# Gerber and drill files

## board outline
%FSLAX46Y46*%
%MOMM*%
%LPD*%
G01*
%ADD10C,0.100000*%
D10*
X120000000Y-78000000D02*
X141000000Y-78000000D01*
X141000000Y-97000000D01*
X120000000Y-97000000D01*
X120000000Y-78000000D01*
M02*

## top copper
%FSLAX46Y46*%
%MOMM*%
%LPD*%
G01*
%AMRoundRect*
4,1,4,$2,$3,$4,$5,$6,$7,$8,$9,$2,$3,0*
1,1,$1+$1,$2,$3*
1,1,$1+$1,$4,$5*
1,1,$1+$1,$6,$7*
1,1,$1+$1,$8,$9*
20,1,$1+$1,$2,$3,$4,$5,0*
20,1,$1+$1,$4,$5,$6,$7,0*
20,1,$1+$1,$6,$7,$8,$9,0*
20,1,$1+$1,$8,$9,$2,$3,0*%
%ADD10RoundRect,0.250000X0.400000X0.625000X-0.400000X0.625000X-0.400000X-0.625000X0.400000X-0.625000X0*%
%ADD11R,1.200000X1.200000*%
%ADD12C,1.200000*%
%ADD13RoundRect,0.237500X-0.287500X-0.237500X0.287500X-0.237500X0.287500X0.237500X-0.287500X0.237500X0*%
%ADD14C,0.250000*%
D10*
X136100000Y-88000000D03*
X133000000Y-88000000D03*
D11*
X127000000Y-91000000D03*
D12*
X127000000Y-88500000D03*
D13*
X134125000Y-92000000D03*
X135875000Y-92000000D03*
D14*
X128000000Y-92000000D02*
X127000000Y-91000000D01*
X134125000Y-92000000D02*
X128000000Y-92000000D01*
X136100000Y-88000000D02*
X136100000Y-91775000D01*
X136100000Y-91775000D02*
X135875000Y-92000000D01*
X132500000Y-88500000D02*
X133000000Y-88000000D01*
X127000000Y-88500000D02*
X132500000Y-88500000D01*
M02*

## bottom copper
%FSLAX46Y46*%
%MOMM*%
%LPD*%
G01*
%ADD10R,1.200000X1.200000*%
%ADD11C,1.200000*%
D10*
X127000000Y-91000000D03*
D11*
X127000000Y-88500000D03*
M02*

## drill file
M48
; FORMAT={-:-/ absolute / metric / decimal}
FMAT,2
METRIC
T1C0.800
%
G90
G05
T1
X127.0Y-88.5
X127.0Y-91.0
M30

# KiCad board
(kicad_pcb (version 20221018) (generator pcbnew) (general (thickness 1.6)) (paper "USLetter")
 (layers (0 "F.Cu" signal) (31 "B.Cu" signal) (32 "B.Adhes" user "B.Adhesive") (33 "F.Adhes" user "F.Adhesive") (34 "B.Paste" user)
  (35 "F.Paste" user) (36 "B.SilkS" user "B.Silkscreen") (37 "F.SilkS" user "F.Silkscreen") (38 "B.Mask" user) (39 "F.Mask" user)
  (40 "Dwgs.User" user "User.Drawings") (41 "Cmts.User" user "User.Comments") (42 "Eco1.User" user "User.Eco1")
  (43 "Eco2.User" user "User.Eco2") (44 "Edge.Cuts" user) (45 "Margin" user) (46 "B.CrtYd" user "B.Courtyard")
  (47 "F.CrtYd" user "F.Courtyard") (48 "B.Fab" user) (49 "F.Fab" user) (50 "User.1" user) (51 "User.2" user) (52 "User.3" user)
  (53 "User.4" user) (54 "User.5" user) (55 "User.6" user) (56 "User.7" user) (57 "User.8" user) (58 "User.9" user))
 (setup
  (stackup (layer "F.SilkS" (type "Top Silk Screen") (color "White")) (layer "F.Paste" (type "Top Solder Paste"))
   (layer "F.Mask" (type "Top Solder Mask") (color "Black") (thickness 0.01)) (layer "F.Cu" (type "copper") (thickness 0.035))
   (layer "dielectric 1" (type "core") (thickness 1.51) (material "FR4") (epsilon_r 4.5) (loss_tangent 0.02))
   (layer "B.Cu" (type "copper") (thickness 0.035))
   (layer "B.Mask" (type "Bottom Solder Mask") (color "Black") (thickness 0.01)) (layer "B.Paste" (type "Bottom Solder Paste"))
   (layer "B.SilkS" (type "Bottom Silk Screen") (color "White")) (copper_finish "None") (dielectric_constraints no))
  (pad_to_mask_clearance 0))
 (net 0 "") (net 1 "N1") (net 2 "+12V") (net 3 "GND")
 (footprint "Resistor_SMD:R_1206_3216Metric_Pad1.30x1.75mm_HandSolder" (layer "F.Cu") (at 134.55 88 180)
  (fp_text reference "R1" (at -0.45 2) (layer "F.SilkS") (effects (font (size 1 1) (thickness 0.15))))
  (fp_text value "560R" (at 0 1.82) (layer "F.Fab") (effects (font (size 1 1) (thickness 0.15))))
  (pad "1" smd roundrect (at -1.55 0 180) (size 1.3 1.75) (layers "F.Cu" "F.Paste" "F.Mask") (roundrect_rratio 0.192308) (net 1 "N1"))
  (pad "2" smd roundrect (at 1.55 0 180) (size 1.3 1.75) (layers "F.Cu" "F.Paste" "F.Mask") (roundrect_rratio 0.192308) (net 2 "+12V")))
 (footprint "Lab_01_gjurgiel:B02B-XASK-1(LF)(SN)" (layer "F.Cu") (at 127 91 90)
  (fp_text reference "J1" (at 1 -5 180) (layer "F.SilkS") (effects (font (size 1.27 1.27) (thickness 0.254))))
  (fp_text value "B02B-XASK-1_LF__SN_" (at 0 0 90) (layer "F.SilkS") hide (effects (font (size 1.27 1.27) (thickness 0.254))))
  (pad "1" thru_hole rect (at 0 0 90) (size 1.2 1.2) (drill 0.8) (layers "*.Cu" "*.Mask") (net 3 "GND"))
  (pad "2" thru_hole circle (at 2.5 0 90) (size 1.2 1.2) (drill 0.8) (layers "*.Cu" "*.Mask") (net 2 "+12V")))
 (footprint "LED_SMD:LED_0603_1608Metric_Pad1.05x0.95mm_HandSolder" (layer "F.Cu") (at 135 92)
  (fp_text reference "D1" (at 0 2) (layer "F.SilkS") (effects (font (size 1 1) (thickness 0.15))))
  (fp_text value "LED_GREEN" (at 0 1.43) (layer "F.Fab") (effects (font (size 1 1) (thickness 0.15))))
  (pad "1" smd roundrect (at -0.875 0) (size 1.05 0.95) (layers "F.Cu" "F.Paste" "F.Mask") (roundrect_rratio 0.25) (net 3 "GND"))
  (pad "2" smd roundrect (at 0.875 0) (size 1.05 0.95) (layers "F.Cu" "F.Paste" "F.Mask") (roundrect_rratio 0.25) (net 1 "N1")))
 (gr_rect (start 120 78) (end 141 97) (stroke (width 0.1) (type default)) (fill none) (layer "Edge.Cuts"))
 (segment (start 128 92) (end 127 91) (width 0.25) (layer "F.Cu") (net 3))
 (segment (start 134.125 92) (end 128 92) (width 0.25) (layer "F.Cu") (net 3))
 (segment (start 136.1 88) (end 136.1 91.775) (width 0.25) (layer "F.Cu") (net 1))
 (segment (start 136.1 91.775) (end 135.875 92) (width 0.25) (layer "F.Cu") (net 1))
 (segment (start 132.5 88.5) (end 133 88) (width 0.25) (layer "F.Cu") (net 2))
 (segment (start 127 88.5) (end 132.5 88.5) (width 0.25) (layer "F.Cu") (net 2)))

